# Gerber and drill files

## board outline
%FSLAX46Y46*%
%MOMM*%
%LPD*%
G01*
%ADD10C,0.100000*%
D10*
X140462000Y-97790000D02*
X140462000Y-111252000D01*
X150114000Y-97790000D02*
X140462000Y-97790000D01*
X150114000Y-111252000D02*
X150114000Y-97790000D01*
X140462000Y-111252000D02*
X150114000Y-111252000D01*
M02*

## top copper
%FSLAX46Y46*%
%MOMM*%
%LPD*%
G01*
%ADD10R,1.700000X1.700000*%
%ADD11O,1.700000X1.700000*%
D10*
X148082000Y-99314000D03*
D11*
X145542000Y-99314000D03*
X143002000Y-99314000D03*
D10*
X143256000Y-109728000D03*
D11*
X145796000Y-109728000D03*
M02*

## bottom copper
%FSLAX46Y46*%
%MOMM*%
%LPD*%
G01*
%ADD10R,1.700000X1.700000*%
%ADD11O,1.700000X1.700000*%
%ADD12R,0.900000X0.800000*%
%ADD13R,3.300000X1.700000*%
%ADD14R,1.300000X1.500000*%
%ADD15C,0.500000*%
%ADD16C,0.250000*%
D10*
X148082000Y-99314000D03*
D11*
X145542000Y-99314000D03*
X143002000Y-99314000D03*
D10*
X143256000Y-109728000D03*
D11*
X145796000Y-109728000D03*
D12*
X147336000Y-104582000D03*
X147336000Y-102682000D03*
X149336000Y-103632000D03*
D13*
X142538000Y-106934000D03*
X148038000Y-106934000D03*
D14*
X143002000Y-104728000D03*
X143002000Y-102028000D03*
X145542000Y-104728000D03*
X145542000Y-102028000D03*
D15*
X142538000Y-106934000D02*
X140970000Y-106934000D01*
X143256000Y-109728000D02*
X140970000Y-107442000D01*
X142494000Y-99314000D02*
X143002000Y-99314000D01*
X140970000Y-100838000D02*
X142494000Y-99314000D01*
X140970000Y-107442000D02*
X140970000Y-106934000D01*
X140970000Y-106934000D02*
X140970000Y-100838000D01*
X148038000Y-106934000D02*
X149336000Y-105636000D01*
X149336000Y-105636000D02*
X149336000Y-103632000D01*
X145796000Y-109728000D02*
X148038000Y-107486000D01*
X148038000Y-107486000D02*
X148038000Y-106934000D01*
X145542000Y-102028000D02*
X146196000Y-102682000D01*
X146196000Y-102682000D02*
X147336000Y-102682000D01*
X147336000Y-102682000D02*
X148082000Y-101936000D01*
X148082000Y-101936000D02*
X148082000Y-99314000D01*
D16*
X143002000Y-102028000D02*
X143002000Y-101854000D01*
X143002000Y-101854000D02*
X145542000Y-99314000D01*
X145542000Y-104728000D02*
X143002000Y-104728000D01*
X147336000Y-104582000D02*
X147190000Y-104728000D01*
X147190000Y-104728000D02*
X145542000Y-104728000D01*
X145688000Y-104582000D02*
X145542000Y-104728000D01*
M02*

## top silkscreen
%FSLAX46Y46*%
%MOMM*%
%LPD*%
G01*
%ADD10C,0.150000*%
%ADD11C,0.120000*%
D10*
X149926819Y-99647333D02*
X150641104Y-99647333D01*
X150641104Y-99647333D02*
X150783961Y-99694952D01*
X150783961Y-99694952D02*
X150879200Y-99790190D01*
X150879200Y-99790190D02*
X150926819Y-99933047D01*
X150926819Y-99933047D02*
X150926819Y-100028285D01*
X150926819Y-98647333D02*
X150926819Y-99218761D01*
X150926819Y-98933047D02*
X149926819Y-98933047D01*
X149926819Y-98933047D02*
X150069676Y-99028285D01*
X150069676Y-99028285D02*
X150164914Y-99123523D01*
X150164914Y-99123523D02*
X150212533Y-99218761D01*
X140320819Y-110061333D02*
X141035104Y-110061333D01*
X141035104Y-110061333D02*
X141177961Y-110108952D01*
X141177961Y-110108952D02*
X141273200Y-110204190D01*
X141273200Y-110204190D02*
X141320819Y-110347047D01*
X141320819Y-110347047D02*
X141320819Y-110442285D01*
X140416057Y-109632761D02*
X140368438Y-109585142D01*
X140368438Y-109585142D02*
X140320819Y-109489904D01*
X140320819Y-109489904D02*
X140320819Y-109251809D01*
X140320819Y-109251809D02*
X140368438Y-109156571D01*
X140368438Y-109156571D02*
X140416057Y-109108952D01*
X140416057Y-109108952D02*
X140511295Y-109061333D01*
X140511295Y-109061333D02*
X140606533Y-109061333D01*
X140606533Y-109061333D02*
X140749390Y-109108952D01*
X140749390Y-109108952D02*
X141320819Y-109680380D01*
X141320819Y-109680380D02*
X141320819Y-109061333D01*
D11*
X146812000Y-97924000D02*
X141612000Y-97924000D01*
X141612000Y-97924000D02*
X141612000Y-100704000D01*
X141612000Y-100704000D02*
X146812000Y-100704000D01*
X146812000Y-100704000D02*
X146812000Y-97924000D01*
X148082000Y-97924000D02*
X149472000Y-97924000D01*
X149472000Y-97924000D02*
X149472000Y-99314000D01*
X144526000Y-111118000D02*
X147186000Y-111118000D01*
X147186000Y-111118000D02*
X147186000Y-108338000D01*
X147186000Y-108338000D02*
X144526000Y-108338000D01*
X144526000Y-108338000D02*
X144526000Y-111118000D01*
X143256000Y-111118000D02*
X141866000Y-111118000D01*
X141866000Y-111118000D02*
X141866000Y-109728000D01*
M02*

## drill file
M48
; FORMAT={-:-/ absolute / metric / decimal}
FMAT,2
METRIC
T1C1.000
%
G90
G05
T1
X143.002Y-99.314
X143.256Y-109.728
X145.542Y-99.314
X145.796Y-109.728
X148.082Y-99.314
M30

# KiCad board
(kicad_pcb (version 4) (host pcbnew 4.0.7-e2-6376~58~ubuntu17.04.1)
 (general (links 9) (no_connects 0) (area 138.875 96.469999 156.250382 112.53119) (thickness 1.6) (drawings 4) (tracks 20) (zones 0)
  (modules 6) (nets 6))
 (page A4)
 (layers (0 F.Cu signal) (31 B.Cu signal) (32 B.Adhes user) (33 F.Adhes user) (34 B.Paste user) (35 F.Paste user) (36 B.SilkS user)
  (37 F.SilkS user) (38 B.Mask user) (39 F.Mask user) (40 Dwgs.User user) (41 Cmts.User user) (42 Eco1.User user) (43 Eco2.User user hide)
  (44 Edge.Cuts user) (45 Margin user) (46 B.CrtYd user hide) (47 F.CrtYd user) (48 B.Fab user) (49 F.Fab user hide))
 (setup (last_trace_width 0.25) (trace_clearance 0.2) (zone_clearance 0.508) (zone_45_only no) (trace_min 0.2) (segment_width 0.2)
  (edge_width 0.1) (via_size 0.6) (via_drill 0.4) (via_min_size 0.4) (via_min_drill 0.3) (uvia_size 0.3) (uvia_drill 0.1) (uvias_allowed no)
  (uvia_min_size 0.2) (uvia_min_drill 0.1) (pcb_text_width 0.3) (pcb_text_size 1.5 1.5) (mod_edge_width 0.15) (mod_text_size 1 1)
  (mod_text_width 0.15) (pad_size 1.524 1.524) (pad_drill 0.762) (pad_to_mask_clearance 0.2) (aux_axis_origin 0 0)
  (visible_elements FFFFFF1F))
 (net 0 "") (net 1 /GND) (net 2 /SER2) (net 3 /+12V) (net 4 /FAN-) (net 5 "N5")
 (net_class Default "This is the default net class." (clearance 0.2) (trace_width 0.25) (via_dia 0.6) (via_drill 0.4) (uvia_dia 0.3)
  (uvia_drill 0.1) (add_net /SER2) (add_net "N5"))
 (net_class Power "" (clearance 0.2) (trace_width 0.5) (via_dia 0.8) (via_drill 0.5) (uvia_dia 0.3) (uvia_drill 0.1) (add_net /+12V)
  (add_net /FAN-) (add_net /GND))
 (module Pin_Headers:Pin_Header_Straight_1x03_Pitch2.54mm (layer F.Cu) (at 148.082 99.314 270)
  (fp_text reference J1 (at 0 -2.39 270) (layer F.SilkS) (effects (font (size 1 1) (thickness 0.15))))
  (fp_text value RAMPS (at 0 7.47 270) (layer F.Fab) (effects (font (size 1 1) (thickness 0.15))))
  (fp_line (start -1.39 1.27) (end -1.39 6.47) (layer F.SilkS) (width 0.12))
  (fp_line (start -1.39 6.47) (end 1.39 6.47) (layer F.SilkS) (width 0.12))
  (fp_line (start 1.39 6.47) (end 1.39 1.27) (layer F.SilkS) (width 0.12))
  (fp_line (start 1.39 1.27) (end -1.39 1.27) (layer F.SilkS) (width 0.12))
  (fp_line (start -1.39 0) (end -1.39 -1.39) (layer F.SilkS) (width 0.12))
  (fp_line (start -1.39 -1.39) (end 0 -1.39) (layer F.SilkS) (width 0.12))
  (pad 1 thru_hole rect (at 0 0 270) (size 1.7 1.7) (drill 1) (layers *.Cu *.Mask) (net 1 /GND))
  (pad 2 thru_hole oval (at 0 2.54 270) (size 1.7 1.7) (drill 1) (layers *.Cu *.Mask) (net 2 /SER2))
  (pad 3 thru_hole oval (at 0 5.08 270) (size 1.7 1.7) (drill 1) (layers *.Cu *.Mask) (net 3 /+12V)))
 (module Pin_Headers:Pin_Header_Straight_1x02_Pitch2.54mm (layer F.Cu) (at 143.256 109.728 90)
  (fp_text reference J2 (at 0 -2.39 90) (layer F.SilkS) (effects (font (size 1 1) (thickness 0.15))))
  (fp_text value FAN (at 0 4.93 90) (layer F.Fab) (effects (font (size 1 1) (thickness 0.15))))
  (fp_line (start -1.39 1.27) (end -1.39 3.93) (layer F.SilkS) (width 0.12))
  (fp_line (start -1.39 3.93) (end 1.39 3.93) (layer F.SilkS) (width 0.12))
  (fp_line (start 1.39 3.93) (end 1.39 1.27) (layer F.SilkS) (width 0.12))
  (fp_line (start 1.39 1.27) (end -1.39 1.27) (layer F.SilkS) (width 0.12))
  (fp_line (start -1.39 0) (end -1.39 -1.39) (layer F.SilkS) (width 0.12))
  (fp_line (start -1.39 -1.39) (end 0 -1.39) (layer F.SilkS) (width 0.12))
  (pad 1 thru_hole rect (at 0 0 90) (size 1.7 1.7) (drill 1) (layers *.Cu *.Mask) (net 3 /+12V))
  (pad 2 thru_hole oval (at 0 2.54 90) (size 1.7 1.7) (drill 1) (layers *.Cu *.Mask) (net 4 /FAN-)))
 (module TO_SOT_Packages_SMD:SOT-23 (layer B.Cu) (at 148.336 103.632)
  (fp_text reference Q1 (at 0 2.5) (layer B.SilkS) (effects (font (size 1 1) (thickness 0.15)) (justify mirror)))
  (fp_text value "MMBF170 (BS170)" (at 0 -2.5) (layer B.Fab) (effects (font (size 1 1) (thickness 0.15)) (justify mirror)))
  (pad 1 smd rect (at -1 0.95) (size 0.9 0.8) (layers B.Cu B.Paste B.Mask) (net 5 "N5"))
  (pad 2 smd rect (at -1 -0.95) (size 0.9 0.8) (layers B.Cu B.Paste B.Mask) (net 1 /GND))
  (pad 3 smd rect (at 1 0) (size 0.9 0.8) (layers B.Cu B.Paste B.Mask) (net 4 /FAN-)))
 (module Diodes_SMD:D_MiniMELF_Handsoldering (layer B.Cu) (at 145.288 106.934)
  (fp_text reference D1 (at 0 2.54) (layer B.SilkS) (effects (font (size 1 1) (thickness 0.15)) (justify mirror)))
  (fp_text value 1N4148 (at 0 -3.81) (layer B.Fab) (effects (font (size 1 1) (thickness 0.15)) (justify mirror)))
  (pad 1 smd rect (at -2.75 0) (size 3.3 1.7) (layers B.Cu B.Paste B.Mask) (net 3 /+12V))
  (pad 2 smd rect (at 2.75 0) (size 3.3 1.7) (layers B.Cu B.Paste B.Mask) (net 4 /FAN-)))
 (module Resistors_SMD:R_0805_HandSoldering (layer B.Cu) (at 143.002 103.378 90)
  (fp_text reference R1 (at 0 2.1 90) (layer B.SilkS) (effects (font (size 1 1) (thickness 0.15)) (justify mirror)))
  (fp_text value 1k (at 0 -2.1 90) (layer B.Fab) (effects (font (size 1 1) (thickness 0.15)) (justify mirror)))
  (pad 1 smd rect (at -1.35 0 90) (size 1.5 1.3) (layers B.Cu B.Paste B.Mask) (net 5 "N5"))
  (pad 2 smd rect (at 1.35 0 90) (size 1.5 1.3) (layers B.Cu B.Paste B.Mask) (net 2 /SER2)))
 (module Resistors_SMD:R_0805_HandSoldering (layer B.Cu) (at 145.542 103.378 90)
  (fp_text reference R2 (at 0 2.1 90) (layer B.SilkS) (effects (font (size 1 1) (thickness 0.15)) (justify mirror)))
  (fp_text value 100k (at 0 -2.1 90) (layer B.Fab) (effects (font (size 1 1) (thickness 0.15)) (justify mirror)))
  (pad 1 smd rect (at -1.35 0 90) (size 1.5 1.3) (layers B.Cu B.Paste B.Mask) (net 5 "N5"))
  (pad 2 smd rect (at 1.35 0 90) (size 1.5 1.3) (layers B.Cu B.Paste B.Mask) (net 1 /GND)))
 (gr_line (start 140.462 97.79) (end 140.462 111.252) (angle 90) (layer Edge.Cuts) (width 0.1))
 (gr_line (start 150.114 97.79) (end 140.462 97.79) (angle 90) (layer Edge.Cuts) (width 0.1))
 (gr_line (start 150.114 111.252) (end 150.114 97.79) (angle 90) (layer Edge.Cuts) (width 0.1))
 (gr_line (start 140.462 111.252) (end 150.114 111.252) (angle 90) (layer Edge.Cuts) (width 0.1))
 (segment (start 142.538 106.934) (end 140.97 106.934) (width 0.5) (layer B.Cu) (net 3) (status 10))
 (segment (start 143.256 109.728) (end 140.97 107.442) (width 0.5) (layer B.Cu) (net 3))
 (segment (start 142.494 99.314) (end 143.002 99.314) (width 0.5) (layer B.Cu) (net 3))
 (segment (start 140.97 100.838) (end 142.494 99.314) (width 0.5) (layer B.Cu) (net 3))
 (segment (start 140.97 107.442) (end 140.97 106.934) (width 0.5) (layer B.Cu) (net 3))
 (segment (start 140.97 106.934) (end 140.97 100.838) (width 0.5) (layer B.Cu) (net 3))
 (segment (start 148.038 106.934) (end 149.336 105.636) (width 0.5) (layer B.Cu) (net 4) (status 400000))
 (segment (start 149.336 105.636) (end 149.336 103.632) (width 0.5) (layer B.Cu) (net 4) (status 800000))
 (segment (start 145.796 109.728) (end 148.038 107.486) (width 0.5) (layer B.Cu) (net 4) (status C00000))
 (segment (start 148.038 107.486) (end 148.038 106.934) (width 0.5) (layer B.Cu) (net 4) (status C00000))
 (segment (start 145.542 102.028) (end 146.196 102.682) (width 0.5) (layer B.Cu) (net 1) (status 400000))
 (segment (start 146.196 102.682) (end 147.336 102.682) (width 0.5) (layer B.Cu) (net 1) (status 800000))
 (segment (start 147.336 102.682) (end 148.082 101.936) (width 0.5) (layer B.Cu) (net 1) (status 400000))
 (segment (start 148.082 101.936) (end 148.082 99.314) (width 0.5) (layer B.Cu) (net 1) (status 800000))
 (segment (start 143.002 102.028) (end 143.002 101.854) (width 0.25) (layer B.Cu) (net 2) (status C00000))
 (segment (start 143.002 101.854) (end 145.542 99.314) (width 0.25) (layer B.Cu) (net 2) (status C00000))
 (segment (start 145.542 104.728) (end 143.002 104.728) (width 0.25) (layer B.Cu) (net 5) (status C00000))
 (segment (start 147.336 104.582) (end 147.19 104.728) (width 0.25) (layer B.Cu) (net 5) (status C00000))
 (segment (start 147.19 104.728) (end 145.542 104.728) (width 0.25) (layer B.Cu) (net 5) (status C00000))
 (segment (start 145.688 104.582) (end 145.542 104.728) (width 0.25) (layer B.Cu) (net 5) (status 30)))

